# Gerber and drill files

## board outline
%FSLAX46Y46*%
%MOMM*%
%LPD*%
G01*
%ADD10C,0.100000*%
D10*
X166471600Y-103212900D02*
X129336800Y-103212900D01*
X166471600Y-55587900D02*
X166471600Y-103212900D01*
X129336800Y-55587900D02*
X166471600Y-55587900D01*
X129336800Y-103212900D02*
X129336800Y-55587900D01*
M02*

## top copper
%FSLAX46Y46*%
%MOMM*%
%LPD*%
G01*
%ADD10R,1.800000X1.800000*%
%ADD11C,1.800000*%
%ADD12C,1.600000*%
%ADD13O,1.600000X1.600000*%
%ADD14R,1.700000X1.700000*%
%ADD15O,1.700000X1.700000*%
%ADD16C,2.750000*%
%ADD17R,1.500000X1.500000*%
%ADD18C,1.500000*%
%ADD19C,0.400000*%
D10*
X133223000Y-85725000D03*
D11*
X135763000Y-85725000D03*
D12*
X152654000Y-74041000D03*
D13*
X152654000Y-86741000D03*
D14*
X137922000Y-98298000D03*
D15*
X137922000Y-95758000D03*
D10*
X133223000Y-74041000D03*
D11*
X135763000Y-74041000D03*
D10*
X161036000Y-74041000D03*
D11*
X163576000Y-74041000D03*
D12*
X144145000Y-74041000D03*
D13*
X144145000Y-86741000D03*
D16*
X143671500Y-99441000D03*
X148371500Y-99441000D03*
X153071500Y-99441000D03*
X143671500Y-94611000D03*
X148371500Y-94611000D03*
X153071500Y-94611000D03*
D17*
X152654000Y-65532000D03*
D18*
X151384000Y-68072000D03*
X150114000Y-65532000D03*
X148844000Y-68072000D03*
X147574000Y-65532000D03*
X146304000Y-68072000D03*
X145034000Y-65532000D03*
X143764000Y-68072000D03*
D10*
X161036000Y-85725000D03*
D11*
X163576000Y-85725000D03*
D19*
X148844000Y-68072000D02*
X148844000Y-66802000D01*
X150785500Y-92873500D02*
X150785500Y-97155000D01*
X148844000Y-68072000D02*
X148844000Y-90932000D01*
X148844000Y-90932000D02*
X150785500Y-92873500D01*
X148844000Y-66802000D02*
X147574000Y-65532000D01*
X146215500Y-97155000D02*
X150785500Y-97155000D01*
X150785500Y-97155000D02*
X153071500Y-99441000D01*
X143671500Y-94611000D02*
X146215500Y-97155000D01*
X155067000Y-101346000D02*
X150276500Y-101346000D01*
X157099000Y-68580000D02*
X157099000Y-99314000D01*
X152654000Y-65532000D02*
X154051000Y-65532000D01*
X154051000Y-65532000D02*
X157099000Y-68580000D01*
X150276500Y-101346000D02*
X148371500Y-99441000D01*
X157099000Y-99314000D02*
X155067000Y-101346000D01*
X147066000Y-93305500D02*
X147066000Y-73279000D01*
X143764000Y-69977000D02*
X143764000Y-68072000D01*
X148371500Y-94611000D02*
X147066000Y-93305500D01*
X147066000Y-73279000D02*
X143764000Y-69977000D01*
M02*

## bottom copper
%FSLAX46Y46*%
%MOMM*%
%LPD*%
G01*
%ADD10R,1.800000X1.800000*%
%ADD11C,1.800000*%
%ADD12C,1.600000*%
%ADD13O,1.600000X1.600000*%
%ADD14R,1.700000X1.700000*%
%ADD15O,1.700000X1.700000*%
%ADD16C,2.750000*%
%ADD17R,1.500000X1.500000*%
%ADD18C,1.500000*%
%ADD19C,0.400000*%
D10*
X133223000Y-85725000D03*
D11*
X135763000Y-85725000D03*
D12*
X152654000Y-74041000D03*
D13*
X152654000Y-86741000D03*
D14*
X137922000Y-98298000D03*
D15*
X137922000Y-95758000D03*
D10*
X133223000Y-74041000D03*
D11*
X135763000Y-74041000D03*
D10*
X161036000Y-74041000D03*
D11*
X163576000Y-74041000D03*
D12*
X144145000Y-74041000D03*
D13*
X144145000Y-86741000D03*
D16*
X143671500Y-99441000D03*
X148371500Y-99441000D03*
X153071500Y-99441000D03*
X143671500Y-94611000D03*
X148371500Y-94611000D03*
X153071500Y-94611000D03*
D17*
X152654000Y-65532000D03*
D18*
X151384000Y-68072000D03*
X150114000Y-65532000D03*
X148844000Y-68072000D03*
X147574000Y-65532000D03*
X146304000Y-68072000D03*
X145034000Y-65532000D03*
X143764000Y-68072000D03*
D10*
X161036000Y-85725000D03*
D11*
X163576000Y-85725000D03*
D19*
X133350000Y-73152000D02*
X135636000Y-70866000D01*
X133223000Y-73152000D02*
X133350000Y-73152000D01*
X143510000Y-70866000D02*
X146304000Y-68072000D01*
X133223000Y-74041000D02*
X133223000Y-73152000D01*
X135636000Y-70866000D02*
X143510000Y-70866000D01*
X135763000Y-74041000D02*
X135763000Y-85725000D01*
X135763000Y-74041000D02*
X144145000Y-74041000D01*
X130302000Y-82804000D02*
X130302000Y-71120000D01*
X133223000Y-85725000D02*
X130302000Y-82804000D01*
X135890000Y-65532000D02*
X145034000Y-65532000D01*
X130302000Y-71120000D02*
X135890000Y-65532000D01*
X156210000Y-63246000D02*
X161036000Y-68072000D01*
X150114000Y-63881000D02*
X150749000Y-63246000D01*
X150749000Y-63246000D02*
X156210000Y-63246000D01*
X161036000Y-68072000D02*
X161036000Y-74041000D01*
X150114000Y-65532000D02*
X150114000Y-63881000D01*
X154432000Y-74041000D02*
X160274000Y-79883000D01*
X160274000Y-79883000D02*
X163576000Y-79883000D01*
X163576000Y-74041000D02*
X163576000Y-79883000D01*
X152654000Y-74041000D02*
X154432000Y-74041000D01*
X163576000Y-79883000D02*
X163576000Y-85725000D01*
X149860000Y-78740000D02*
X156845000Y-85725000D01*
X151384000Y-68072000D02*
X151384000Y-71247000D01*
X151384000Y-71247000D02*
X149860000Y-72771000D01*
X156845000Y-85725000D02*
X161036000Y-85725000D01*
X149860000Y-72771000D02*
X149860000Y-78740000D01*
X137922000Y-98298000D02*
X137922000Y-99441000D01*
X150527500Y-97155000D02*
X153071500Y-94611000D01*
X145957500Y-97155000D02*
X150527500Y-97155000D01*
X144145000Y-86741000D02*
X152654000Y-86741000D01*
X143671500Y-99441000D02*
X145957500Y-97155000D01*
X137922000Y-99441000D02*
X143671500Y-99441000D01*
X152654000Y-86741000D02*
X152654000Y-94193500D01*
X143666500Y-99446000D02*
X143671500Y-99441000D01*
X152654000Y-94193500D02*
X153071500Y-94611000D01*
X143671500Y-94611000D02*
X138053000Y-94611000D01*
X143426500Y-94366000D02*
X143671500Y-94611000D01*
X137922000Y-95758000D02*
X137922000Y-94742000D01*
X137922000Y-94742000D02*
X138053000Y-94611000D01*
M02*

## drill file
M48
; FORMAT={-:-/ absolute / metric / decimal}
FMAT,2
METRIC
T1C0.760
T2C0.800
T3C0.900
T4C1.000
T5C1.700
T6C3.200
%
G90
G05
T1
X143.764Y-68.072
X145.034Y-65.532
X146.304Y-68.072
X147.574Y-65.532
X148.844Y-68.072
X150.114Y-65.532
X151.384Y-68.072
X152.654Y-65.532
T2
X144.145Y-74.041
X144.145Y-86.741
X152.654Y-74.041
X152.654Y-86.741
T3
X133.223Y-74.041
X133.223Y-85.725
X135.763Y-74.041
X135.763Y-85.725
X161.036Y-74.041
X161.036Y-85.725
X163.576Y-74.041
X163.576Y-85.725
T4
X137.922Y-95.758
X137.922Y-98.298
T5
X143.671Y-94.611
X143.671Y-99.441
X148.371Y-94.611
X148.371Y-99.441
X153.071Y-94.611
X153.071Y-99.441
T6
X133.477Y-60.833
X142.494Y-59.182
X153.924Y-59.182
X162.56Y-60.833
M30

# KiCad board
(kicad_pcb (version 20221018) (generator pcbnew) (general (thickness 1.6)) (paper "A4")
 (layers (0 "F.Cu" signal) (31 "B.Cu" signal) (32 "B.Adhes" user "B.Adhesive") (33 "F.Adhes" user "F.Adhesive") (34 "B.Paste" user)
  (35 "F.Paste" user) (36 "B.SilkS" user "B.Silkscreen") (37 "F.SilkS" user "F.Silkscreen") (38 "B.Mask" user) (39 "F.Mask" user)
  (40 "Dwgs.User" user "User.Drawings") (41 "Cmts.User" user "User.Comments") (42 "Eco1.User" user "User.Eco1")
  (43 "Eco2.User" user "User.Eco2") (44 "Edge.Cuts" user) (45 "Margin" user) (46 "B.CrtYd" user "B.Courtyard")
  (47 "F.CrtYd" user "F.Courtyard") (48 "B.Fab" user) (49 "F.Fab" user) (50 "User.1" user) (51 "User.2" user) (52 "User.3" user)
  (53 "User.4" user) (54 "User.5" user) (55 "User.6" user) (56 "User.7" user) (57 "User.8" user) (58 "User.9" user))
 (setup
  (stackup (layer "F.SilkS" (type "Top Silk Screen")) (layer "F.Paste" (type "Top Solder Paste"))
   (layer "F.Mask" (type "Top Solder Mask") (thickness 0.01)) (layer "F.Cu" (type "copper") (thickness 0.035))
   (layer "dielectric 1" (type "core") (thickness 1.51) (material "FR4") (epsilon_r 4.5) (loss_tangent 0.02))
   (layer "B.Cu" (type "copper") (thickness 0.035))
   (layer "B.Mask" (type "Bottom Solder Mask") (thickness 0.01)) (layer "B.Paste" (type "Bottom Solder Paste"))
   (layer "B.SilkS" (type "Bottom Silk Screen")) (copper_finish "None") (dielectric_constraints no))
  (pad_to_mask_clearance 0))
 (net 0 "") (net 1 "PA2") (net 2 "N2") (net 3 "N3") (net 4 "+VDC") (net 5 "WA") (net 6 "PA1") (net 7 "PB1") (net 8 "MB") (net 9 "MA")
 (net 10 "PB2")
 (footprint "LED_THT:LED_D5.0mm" (layer "F.Cu") (at 133.223 85.725)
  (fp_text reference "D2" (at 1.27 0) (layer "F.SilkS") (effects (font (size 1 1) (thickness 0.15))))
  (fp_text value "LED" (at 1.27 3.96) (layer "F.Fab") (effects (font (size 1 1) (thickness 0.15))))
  (pad "1" thru_hole rect (at 0 0) (size 1.8 1.8) (drill 0.9) (layers "*.Cu" "*.Mask") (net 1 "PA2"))
  (pad "2" thru_hole circle (at 2.54 0) (size 1.8 1.8) (drill 0.9) (layers "*.Cu" "*.Mask") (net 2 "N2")))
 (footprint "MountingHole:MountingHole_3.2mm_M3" (layer "F.Cu") (at 162.56 60.833)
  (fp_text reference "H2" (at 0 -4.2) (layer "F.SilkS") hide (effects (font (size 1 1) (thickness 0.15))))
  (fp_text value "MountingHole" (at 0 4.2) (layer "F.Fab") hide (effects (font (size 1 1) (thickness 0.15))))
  (pad "" np_thru_hole circle (at 0 0) (size 3.2 3.2) (drill 3.2) (layers "*.Cu" "*.Mask")))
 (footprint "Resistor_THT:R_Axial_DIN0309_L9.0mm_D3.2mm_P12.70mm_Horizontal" (layer "F.Cu") (at 152.654 74.041 -90)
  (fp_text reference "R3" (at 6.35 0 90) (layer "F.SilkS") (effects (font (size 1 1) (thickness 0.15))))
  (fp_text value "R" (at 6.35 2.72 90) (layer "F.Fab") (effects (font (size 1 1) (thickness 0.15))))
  (pad "1" thru_hole circle (at 0 0 270) (size 1.6 1.6) (drill 0.8) (layers "*.Cu" "*.Mask") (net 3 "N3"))
  (pad "2" thru_hole oval (at 12.7 0 270) (size 1.6 1.6) (drill 0.8) (layers "*.Cu" "*.Mask") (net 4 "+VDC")))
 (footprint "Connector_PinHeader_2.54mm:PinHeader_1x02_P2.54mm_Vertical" (layer "F.Cu") (at 137.922 98.298 180)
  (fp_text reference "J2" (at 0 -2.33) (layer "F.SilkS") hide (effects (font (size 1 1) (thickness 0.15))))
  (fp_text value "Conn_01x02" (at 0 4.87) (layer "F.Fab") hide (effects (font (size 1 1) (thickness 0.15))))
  (pad "1" thru_hole rect (at 0 0 180) (size 1.7 1.7) (drill 1) (layers "*.Cu" "*.Mask") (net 4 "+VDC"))
  (pad "2" thru_hole oval (at 0 2.54 180) (size 1.7 1.7) (drill 1) (layers "*.Cu" "*.Mask") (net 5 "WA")))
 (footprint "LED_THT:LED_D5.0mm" (layer "F.Cu") (at 133.223 74.041)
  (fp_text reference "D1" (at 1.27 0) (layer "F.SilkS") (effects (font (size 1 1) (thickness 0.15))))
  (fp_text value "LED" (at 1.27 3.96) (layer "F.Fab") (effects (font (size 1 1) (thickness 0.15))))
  (pad "1" thru_hole rect (at 0 0) (size 1.8 1.8) (drill 0.9) (layers "*.Cu" "*.Mask") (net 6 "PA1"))
  (pad "2" thru_hole circle (at 2.54 0) (size 1.8 1.8) (drill 0.9) (layers "*.Cu" "*.Mask") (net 2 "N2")))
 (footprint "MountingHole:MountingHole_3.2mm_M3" (layer "F.Cu") (at 133.477 60.833)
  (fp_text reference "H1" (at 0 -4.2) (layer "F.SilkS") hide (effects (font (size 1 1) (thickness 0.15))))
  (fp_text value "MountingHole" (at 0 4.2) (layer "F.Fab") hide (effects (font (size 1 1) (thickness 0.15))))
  (pad "" np_thru_hole circle (at 0 0) (size 3.2 3.2) (drill 3.2) (layers "*.Cu" "*.Mask")))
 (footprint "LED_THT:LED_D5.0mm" (layer "F.Cu") (at 161.036 74.041)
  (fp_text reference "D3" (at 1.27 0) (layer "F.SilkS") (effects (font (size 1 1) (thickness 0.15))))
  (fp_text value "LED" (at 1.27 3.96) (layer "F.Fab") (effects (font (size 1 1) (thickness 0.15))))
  (pad "1" thru_hole rect (at 0 0) (size 1.8 1.8) (drill 0.9) (layers "*.Cu" "*.Mask") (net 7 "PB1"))
  (pad "2" thru_hole circle (at 2.54 0) (size 1.8 1.8) (drill 0.9) (layers "*.Cu" "*.Mask") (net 3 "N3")))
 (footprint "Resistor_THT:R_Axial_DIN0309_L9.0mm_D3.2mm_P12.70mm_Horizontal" (layer "F.Cu") (at 144.145 74.041 -90)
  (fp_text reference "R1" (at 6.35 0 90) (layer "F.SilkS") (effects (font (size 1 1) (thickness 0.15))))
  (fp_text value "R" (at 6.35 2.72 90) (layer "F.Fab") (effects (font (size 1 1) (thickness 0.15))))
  (pad "1" thru_hole circle (at 0 0 270) (size 1.6 1.6) (drill 0.8) (layers "*.Cu" "*.Mask") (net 2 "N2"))
  (pad "2" thru_hole oval (at 12.7 0 270) (size 1.6 1.6) (drill 0.8) (layers "*.Cu" "*.Mask") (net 4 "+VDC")))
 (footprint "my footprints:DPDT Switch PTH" (layer "F.Cu") (at 148.3715 97.026 90)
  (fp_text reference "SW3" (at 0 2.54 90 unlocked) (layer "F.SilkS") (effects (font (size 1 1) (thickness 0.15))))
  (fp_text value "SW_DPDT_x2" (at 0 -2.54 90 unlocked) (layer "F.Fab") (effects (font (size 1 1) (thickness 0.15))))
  (pad "1" thru_hole circle (at -2.415 -4.7 90) (size 2.75 2.75) (drill 1.7) (layers "*.Cu" "*.Mask") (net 4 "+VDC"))
  (pad "2" thru_hole circle (at -2.415 0 90) (size 2.75 2.75) (drill 1.7) (layers "*.Cu" "*.Mask") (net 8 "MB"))
  (pad "3" thru_hole circle (at -2.415 4.7 90) (size 2.75 2.75) (drill 1.7) (layers "*.Cu" "*.Mask") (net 5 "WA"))
  (pad "4" thru_hole circle (at 2.415 -4.7 90) (size 2.75 2.75) (drill 1.7) (layers "*.Cu" "*.Mask") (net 5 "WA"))
  (pad "5" thru_hole circle (at 2.415 0 90) (size 2.75 2.75) (drill 1.7) (layers "*.Cu" "*.Mask") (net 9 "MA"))
  (pad "6" thru_hole circle (at 2.415 4.7 90) (size 2.75 2.75) (drill 1.7) (layers "*.Cu" "*.Mask") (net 4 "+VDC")))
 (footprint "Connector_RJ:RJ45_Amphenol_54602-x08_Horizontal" (layer "F.Cu") (at 152.654 65.532 180)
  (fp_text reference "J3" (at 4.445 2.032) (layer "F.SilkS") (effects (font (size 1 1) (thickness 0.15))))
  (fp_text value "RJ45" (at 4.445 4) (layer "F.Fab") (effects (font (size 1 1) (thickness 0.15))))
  (pad "" np_thru_hole circle (at -1.27 6.35 180) (size 3.2 3.2) (drill 3.2) (layers "*.Cu" "*.Mask"))
  (pad "" np_thru_hole circle (at 10.16 6.35 180) (size 3.2 3.2) (drill 3.2) (layers "*.Cu" "*.Mask"))
  (pad "1" thru_hole rect (at 0 0 180) (size 1.5 1.5) (drill 0.76) (layers "*.Cu" "*.Mask") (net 8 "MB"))
  (pad "2" thru_hole circle (at 1.27 -2.54 180) (size 1.5 1.5) (drill 0.76) (layers "*.Cu" "*.Mask") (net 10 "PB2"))
  (pad "3" thru_hole circle (at 2.54 0 180) (size 1.5 1.5) (drill 0.76) (layers "*.Cu" "*.Mask") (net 7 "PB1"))
  (pad "4" thru_hole circle (at 3.81 -2.54 180) (size 1.5 1.5) (drill 0.76) (layers "*.Cu" "*.Mask") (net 5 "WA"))
  (pad "5" thru_hole circle (at 5.08 0 180) (size 1.5 1.5) (drill 0.76) (layers "*.Cu" "*.Mask") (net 5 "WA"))
  (pad "6" thru_hole circle (at 6.35 -2.54 180) (size 1.5 1.5) (drill 0.76) (layers "*.Cu" "*.Mask") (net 6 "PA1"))
  (pad "7" thru_hole circle (at 7.62 0 180) (size 1.5 1.5) (drill 0.76) (layers "*.Cu" "*.Mask") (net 1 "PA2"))
  (pad "8" thru_hole circle (at 8.89 -2.54 180) (size 1.5 1.5) (drill 0.76) (layers "*.Cu" "*.Mask") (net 9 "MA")))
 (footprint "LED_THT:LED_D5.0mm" (layer "F.Cu") (at 161.036 85.725)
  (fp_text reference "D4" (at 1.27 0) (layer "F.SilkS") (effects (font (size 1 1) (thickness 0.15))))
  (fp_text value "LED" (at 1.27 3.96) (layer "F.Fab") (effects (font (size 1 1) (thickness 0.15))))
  (pad "1" thru_hole rect (at 0 0) (size 1.8 1.8) (drill 0.9) (layers "*.Cu" "*.Mask") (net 10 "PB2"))
  (pad "2" thru_hole circle (at 2.54 0) (size 1.8 1.8) (drill 0.9) (layers "*.Cu" "*.Mask") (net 3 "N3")))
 (gr_line (start 166.4716 103.2129) (end 129.3368 103.2129) (stroke (width 0.1) (type default)) (layer "Edge.Cuts"))
 (gr_line (start 166.4716 55.5879) (end 166.4716 103.2129) (stroke (width 0.1) (type default)) (layer "Edge.Cuts"))
 (gr_line (start 129.3368 55.5879) (end 166.4716 55.5879) (stroke (width 0.1) (type default)) (layer "Edge.Cuts"))
 (gr_line (start 129.3368 103.2129) (end 129.3368 55.5879) (stroke (width 0.1) (type default)) (layer "Edge.Cuts"))
 (segment (start 133.35 73.152) (end 135.636 70.866) (width 0.4) (layer "B.Cu") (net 6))
 (segment (start 133.223 73.152) (end 133.35 73.152) (width 0.4) (layer "B.Cu") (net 6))
 (segment (start 143.51 70.866) (end 146.304 68.072) (width 0.4) (layer "B.Cu") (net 6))
 (segment (start 133.223 74.041) (end 133.223 73.152) (width 0.4) (layer "B.Cu") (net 6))
 (segment (start 135.636 70.866) (end 143.51 70.866) (width 0.4) (layer "B.Cu") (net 6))
 (segment (start 135.763 74.041) (end 135.763 85.725) (width 0.4) (layer "B.Cu") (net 2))
 (segment (start 135.763 74.041) (end 144.145 74.041) (width 0.4) (layer "B.Cu") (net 2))
 (segment (start 130.302 82.804) (end 130.302 71.12) (width 0.4) (layer "B.Cu") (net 1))
 (segment (start 133.223 85.725) (end 130.302 82.804) (width 0.4) (layer "B.Cu") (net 1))
 (segment (start 135.89 65.532) (end 145.034 65.532) (width 0.4) (layer "B.Cu") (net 1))
 (segment (start 130.302 71.12) (end 135.89 65.532) (width 0.4) (layer "B.Cu") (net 1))
 (segment (start 156.21 63.246) (end 161.036 68.072) (width 0.4) (layer "B.Cu") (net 7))
 (segment (start 150.114 63.881) (end 150.749 63.246) (width 0.4) (layer "B.Cu") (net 7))
 (segment (start 150.749 63.246) (end 156.21 63.246) (width 0.4) (layer "B.Cu") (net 7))
 (segment (start 161.036 68.072) (end 161.036 74.041) (width 0.4) (layer "B.Cu") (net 7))
 (segment (start 150.114 65.532) (end 150.114 63.881) (width 0.4) (layer "B.Cu") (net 7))
 (segment (start 154.432 74.041) (end 160.274 79.883) (width 0.4) (layer "B.Cu") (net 3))
 (segment (start 160.274 79.883) (end 163.576 79.883) (width 0.4) (layer "B.Cu") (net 3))
 (segment (start 163.576 74.041) (end 163.576 79.883) (width 0.4) (layer "B.Cu") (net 3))
 (segment (start 152.654 74.041) (end 154.432 74.041) (width 0.4) (layer "B.Cu") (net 3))
 (segment (start 163.576 79.883) (end 163.576 85.725) (width 0.4) (layer "B.Cu") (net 3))
 (segment (start 149.86 78.74) (end 156.845 85.725) (width 0.4) (layer "B.Cu") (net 10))
 (segment (start 151.384 68.072) (end 151.384 71.247) (width 0.4) (layer "B.Cu") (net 10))
 (segment (start 151.384 71.247) (end 149.86 72.771) (width 0.4) (layer "B.Cu") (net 10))
 (segment (start 156.845 85.725) (end 161.036 85.725) (width 0.4) (layer "B.Cu") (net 10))
 (segment (start 149.86 72.771) (end 149.86 78.74) (width 0.4) (layer "B.Cu") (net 10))
 (segment (start 137.922 98.298) (end 137.922 99.441) (width 0.4) (layer "B.Cu") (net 4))
 (segment (start 150.5275 97.155) (end 153.0715 94.611) (width 0.4) (layer "B.Cu") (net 4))
 (segment (start 145.9575 97.155) (end 150.5275 97.155) (width 0.4) (layer "B.Cu") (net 4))
 (segment (start 144.145 86.741) (end 152.654 86.741) (width 0.4) (layer "B.Cu") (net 4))
 (segment (start 143.6715 99.441) (end 145.9575 97.155) (width 0.4) (layer "B.Cu") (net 4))
 (segment (start 137.922 99.441) (end 143.6715 99.441) (width 0.4) (layer "B.Cu") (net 4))
 (segment (start 152.654 86.741) (end 152.654 94.1935) (width 0.4) (layer "B.Cu") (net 4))
 (segment (start 143.6665 99.446) (end 143.6715 99.441) (width 0.4) (layer "B.Cu") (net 4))
 (segment (start 152.654 94.1935) (end 153.0715 94.611) (width 0.4) (layer "B.Cu") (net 4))
 (segment (start 148.844 68.072) (end 148.844 66.802) (width 0.4) (layer "F.Cu") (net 5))
 (segment (start 150.7855 92.8735) (end 150.7855 97.155) (width 0.4) (layer "F.Cu") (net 5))
 (segment (start 148.844 68.072) (end 148.844 90.932) (width 0.4) (layer "F.Cu") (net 5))
 (segment (start 148.844 90.932) (end 150.7855 92.8735) (width 0.4) (layer "F.Cu") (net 5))
 (segment (start 148.844 66.802) (end 147.574 65.532) (width 0.4) (layer "F.Cu") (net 5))
 (segment (start 146.2155 97.155) (end 150.7855 97.155) (width 0.4) (layer "F.Cu") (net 5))
 (segment (start 150.7855 97.155) (end 153.0715 99.441) (width 0.4) (layer "F.Cu") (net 5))
 (segment (start 143.6715 94.611) (end 146.2155 97.155) (width 0.4) (layer "F.Cu") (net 5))
 (segment (start 143.6715 94.611) (end 138.053 94.611) (width 0.4) (layer "B.Cu") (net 5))
 (segment (start 143.4265 94.366) (end 143.6715 94.611) (width 0.4) (layer "B.Cu") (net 5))
 (segment (start 137.922 95.758) (end 137.922 94.742) (width 0.4) (layer "B.Cu") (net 5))
 (segment (start 137.922 94.742) (end 138.053 94.611) (width 0.4) (layer "B.Cu") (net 5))
 (segment (start 155.067 101.346) (end 150.2765 101.346) (width 0.4) (layer "F.Cu") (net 8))
 (segment (start 157.099 68.58) (end 157.099 99.314) (width 0.4) (layer "F.Cu") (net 8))
 (segment (start 152.654 65.532) (end 154.051 65.532) (width 0.4) (layer "F.Cu") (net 8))
 (segment (start 154.051 65.532) (end 157.099 68.58) (width 0.4) (layer "F.Cu") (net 8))
 (segment (start 150.2765 101.346) (end 148.3715 99.441) (width 0.4) (layer "F.Cu") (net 8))
 (segment (start 157.099 99.314) (end 155.067 101.346) (width 0.4) (layer "F.Cu") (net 8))
 (segment (start 147.066 93.3055) (end 147.066 73.279) (width 0.4) (layer "F.Cu") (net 9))
 (segment (start 143.764 69.977) (end 143.764 68.072) (width 0.4) (layer "F.Cu") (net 9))
 (segment (start 148.3715 94.611) (end 147.066 93.3055) (width 0.4) (layer "F.Cu") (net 9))
 (segment (start 147.066 73.279) (end 143.764 69.977) (width 0.4) (layer "F.Cu") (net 9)))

